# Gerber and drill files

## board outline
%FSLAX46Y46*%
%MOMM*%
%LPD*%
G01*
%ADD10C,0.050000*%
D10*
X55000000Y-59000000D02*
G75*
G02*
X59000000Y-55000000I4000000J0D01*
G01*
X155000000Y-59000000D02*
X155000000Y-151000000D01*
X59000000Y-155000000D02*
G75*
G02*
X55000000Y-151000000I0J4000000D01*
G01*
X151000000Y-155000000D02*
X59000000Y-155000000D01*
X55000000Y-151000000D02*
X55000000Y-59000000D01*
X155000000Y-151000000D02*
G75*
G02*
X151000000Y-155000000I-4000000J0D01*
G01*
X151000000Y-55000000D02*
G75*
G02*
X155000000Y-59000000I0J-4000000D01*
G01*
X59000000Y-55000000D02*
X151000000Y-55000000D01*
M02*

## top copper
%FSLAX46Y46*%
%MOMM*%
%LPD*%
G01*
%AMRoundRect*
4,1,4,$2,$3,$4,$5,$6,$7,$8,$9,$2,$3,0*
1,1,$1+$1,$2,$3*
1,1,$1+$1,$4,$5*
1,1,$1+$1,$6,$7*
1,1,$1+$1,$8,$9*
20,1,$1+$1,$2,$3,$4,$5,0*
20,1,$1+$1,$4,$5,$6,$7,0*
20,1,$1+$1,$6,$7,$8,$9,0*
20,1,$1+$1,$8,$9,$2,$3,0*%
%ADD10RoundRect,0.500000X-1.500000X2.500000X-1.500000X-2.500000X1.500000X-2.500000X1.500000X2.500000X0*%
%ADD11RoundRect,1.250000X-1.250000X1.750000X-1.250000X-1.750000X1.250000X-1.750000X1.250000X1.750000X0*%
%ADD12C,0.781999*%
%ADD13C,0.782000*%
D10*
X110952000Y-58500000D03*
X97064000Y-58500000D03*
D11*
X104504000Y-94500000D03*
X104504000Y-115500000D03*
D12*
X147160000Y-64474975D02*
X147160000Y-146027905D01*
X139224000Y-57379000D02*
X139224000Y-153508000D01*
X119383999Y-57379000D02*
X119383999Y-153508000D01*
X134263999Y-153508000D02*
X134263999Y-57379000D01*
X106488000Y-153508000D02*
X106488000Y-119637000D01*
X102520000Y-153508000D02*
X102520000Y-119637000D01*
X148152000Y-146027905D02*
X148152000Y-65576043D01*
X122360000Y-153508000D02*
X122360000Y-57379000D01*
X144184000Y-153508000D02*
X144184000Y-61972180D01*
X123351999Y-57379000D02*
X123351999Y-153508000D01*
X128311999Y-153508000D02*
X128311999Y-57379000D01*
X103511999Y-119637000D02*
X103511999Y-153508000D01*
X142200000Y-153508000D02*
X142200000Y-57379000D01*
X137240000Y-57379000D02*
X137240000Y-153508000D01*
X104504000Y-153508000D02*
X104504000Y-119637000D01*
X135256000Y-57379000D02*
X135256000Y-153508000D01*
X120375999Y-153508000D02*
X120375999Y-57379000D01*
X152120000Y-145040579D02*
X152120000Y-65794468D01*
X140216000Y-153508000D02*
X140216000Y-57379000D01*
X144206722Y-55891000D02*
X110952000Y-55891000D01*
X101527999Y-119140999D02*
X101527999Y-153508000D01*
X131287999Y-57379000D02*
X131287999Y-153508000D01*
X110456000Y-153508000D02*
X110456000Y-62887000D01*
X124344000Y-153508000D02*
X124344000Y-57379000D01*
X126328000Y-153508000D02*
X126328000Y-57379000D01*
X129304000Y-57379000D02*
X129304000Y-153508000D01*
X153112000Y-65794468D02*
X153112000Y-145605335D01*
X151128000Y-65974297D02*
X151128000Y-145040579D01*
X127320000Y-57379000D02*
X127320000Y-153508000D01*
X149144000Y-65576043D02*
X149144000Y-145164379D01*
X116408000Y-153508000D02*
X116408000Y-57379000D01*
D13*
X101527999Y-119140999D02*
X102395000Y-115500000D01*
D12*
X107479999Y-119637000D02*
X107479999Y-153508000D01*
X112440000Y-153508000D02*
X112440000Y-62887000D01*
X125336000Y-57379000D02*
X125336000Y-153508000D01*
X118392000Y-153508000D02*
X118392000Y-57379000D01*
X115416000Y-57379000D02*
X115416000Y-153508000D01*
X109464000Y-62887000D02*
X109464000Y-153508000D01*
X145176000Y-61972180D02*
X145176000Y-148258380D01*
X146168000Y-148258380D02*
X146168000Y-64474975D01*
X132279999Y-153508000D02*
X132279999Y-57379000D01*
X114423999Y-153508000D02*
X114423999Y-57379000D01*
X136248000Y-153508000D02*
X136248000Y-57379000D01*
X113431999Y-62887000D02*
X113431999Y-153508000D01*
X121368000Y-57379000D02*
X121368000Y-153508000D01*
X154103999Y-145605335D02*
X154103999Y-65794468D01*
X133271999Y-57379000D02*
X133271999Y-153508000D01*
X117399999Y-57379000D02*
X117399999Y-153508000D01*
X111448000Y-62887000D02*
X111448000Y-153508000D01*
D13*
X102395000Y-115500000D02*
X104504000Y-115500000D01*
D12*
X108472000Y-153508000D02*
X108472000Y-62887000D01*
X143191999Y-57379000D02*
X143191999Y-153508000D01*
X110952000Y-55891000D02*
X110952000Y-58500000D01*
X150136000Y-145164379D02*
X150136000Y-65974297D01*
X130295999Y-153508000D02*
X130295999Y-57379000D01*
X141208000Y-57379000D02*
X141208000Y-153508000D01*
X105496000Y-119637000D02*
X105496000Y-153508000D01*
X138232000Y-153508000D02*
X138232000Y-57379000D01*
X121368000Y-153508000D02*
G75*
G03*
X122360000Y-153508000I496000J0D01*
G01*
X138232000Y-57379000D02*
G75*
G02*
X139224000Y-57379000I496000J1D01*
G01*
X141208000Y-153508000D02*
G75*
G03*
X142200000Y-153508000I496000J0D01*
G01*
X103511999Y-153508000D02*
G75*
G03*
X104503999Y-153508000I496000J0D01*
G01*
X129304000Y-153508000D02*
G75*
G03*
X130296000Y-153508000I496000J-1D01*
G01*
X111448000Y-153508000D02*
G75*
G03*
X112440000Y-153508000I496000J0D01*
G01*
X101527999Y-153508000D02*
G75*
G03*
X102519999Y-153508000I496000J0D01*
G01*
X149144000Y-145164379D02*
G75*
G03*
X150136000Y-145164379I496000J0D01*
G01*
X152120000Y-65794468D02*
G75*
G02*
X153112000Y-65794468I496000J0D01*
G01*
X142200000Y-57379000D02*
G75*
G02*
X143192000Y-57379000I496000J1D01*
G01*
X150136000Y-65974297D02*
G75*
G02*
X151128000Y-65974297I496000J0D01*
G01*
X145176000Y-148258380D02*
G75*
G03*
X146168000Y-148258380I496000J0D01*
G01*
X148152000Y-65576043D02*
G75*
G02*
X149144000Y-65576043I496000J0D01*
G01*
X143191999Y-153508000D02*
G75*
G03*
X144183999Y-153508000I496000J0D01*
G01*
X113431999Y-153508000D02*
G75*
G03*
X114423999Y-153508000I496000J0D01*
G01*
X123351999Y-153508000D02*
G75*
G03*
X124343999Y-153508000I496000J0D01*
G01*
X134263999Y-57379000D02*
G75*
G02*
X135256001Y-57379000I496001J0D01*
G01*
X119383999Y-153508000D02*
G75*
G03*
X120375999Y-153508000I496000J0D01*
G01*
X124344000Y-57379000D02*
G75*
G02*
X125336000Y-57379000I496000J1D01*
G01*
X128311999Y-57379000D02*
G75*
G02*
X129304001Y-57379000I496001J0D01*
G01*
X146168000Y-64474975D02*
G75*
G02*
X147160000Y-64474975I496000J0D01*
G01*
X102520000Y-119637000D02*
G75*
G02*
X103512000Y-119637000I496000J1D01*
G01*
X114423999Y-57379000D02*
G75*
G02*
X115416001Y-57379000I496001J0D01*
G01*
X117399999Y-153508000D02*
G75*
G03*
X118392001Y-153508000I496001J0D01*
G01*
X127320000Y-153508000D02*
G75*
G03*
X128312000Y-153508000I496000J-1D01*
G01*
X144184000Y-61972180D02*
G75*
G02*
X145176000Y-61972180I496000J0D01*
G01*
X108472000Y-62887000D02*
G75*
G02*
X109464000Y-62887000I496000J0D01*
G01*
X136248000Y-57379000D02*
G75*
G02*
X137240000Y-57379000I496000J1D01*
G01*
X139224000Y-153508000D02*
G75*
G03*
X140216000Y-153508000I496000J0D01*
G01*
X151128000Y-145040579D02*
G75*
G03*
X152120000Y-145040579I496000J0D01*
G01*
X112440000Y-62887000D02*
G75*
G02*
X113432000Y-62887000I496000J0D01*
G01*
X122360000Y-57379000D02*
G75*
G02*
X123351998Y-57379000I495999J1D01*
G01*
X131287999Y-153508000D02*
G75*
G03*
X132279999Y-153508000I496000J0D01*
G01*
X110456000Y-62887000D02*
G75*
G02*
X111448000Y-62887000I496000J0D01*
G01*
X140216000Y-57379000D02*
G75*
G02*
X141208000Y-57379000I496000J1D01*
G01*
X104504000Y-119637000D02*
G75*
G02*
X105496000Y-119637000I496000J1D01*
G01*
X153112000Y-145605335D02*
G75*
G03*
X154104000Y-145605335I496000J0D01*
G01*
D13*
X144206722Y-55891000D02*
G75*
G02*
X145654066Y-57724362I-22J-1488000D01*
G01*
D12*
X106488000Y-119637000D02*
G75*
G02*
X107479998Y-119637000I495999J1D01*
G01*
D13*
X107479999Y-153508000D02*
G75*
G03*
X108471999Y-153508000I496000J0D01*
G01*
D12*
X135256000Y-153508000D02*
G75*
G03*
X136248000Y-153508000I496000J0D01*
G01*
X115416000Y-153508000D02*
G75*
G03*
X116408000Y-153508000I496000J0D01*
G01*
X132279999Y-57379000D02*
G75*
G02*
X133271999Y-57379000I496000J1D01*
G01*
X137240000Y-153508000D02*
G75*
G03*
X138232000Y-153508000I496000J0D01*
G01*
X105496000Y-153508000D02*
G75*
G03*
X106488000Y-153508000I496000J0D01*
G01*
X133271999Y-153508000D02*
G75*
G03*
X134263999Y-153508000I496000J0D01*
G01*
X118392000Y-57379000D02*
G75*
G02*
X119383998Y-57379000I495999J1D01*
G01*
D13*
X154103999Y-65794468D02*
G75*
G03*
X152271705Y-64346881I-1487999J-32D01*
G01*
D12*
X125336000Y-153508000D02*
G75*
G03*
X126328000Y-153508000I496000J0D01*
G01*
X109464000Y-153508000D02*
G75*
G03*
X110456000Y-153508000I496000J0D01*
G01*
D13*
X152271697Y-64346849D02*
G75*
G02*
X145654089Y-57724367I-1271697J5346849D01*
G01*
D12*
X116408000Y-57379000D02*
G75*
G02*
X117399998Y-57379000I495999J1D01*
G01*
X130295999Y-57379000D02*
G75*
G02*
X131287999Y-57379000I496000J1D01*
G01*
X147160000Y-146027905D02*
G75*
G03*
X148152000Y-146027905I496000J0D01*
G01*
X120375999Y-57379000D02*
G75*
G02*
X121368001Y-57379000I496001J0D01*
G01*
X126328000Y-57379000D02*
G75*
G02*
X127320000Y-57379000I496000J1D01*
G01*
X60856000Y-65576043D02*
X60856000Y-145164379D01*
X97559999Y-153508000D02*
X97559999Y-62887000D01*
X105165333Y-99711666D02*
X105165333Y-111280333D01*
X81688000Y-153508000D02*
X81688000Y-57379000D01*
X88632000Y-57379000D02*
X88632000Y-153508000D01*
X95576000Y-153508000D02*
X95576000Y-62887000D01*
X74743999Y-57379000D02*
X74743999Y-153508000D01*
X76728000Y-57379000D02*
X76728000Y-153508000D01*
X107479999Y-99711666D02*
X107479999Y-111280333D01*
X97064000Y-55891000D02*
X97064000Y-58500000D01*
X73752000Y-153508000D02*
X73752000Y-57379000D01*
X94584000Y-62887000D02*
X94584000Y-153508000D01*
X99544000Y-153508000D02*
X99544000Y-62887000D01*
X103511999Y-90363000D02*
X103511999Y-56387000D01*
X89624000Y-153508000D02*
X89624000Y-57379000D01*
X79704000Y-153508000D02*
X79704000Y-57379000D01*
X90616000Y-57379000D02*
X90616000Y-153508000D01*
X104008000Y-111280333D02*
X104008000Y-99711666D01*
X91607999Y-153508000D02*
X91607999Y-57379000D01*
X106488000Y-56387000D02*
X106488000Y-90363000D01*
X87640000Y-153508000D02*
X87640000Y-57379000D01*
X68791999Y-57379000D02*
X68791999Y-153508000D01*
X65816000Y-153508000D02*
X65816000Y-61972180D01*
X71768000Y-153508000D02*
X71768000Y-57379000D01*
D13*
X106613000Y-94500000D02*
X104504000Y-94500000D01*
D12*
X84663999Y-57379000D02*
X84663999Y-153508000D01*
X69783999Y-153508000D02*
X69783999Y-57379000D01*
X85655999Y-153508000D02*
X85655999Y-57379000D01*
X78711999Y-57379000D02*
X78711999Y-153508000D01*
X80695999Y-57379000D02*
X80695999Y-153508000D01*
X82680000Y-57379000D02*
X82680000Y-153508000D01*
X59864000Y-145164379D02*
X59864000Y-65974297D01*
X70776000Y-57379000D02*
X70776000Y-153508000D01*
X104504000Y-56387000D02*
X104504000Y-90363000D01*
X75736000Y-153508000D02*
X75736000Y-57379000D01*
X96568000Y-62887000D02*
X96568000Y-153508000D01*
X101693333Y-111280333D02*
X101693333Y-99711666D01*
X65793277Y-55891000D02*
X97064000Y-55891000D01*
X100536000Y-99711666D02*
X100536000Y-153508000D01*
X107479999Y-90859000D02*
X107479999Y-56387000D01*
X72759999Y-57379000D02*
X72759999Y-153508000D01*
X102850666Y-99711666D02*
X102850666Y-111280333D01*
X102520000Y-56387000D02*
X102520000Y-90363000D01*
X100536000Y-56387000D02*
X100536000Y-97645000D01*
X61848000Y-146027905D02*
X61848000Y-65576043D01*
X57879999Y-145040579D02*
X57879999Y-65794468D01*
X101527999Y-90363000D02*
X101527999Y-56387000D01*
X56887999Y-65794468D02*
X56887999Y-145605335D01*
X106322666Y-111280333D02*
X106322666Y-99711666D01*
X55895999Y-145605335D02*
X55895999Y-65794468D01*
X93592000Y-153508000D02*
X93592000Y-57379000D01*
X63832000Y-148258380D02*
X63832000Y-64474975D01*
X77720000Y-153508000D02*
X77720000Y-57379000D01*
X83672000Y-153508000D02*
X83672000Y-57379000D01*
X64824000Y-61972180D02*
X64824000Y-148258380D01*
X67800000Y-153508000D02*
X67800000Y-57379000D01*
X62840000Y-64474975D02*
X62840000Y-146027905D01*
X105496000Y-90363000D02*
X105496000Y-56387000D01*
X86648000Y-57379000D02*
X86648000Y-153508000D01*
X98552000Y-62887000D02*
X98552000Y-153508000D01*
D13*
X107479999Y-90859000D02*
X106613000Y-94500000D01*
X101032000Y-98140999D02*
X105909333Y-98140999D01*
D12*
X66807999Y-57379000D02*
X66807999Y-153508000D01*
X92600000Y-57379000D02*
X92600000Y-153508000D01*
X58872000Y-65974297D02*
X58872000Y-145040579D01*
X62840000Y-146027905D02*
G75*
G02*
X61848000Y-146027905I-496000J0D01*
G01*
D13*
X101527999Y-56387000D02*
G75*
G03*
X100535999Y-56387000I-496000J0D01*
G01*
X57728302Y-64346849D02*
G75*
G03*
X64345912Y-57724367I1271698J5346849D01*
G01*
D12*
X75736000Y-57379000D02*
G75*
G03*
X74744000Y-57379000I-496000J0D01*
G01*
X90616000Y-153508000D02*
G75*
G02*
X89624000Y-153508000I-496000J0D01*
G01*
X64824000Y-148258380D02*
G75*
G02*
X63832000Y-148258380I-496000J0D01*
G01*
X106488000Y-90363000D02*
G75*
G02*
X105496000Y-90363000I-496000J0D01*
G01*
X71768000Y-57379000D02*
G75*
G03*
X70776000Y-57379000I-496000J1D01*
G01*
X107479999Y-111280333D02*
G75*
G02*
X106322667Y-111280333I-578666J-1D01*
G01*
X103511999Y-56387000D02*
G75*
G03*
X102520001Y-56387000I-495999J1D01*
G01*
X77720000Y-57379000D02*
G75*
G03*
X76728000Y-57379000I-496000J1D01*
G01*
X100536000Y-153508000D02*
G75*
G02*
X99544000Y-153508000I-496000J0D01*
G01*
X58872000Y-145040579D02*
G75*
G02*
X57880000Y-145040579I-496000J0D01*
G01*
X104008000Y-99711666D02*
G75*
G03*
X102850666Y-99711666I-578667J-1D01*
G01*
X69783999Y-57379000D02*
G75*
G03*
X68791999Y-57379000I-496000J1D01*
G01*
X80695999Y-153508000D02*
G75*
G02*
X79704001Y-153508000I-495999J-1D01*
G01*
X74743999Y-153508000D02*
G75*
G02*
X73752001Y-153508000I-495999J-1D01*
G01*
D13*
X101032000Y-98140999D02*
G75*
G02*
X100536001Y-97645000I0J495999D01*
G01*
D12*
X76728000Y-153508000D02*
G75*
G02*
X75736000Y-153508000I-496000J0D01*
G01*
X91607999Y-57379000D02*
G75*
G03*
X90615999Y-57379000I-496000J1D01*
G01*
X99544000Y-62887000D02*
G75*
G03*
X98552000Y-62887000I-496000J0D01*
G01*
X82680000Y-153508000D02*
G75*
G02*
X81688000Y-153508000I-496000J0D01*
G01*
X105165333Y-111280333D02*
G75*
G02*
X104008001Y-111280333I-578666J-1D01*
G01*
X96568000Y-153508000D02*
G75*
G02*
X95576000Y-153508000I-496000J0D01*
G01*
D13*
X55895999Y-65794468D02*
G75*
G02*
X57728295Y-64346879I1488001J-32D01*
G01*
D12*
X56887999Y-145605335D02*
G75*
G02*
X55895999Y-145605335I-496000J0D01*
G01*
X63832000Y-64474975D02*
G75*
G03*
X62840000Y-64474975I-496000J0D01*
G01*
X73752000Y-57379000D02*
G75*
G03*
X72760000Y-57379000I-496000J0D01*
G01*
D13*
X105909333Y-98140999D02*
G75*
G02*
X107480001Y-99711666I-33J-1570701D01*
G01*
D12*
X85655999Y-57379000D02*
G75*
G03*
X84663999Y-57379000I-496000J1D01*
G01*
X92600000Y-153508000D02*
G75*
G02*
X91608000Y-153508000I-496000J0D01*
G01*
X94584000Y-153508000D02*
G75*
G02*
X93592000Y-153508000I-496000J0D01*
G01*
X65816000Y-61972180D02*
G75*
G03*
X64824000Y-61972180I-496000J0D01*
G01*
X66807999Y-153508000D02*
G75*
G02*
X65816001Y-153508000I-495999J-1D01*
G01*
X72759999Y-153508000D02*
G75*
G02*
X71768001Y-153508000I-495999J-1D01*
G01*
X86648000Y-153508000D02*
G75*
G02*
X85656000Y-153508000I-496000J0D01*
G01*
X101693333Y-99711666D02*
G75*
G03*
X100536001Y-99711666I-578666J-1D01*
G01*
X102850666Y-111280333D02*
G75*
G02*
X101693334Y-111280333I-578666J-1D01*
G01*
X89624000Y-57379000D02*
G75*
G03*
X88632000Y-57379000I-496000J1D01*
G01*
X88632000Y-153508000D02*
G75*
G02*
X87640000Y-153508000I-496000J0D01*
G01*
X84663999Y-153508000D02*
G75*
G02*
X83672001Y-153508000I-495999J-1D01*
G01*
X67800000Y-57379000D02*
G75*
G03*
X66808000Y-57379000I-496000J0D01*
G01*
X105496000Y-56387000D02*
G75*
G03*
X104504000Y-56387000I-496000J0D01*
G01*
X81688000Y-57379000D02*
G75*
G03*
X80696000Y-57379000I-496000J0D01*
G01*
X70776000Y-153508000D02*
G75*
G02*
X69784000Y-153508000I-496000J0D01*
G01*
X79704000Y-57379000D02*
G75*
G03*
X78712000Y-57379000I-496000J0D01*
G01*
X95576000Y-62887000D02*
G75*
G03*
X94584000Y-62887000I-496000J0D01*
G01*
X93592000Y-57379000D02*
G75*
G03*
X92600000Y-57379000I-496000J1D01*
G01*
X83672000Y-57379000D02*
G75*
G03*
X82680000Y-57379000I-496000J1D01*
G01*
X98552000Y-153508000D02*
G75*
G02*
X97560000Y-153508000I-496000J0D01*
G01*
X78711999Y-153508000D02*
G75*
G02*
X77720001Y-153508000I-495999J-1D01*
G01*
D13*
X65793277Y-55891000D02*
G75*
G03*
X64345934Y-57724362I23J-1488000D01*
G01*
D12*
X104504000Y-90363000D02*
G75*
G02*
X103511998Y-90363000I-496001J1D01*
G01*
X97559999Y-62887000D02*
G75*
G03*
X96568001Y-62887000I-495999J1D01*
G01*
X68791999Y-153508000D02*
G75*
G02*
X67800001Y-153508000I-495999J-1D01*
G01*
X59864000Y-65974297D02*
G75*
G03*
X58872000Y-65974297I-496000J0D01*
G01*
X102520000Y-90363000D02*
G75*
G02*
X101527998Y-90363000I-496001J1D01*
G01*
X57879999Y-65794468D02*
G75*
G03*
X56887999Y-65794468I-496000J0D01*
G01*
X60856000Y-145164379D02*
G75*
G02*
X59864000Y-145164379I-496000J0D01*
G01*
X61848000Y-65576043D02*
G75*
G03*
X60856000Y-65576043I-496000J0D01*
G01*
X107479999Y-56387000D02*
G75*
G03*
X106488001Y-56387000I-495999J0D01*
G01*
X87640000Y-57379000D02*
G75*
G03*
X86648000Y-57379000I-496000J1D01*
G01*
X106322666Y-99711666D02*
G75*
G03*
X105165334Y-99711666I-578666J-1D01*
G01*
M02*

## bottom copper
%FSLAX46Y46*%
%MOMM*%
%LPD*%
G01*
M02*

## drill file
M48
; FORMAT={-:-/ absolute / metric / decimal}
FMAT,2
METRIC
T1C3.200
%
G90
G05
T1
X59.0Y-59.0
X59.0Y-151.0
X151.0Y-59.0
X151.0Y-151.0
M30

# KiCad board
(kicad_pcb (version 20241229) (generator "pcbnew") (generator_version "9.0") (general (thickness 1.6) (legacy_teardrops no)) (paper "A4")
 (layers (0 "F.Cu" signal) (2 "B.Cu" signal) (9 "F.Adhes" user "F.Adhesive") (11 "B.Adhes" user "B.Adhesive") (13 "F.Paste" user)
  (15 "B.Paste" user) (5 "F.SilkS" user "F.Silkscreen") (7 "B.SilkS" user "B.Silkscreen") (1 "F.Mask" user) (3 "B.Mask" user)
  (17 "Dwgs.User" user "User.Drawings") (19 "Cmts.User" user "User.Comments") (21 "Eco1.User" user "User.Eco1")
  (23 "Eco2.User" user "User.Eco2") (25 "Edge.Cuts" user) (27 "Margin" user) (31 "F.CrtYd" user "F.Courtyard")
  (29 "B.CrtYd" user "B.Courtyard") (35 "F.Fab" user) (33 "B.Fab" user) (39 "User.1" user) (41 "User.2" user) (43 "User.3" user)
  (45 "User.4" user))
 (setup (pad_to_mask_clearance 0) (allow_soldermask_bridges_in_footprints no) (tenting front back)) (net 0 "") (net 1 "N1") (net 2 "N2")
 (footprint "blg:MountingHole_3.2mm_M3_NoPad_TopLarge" (layer "F.Cu") (at 151 59)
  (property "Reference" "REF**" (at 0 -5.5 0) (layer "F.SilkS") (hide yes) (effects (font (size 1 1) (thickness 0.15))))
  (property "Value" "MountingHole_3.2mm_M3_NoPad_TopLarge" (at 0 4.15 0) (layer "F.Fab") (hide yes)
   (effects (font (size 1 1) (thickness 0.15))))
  (pad "" np_thru_hole circle (at 0 0) (size 7.6 7.6) (drill 3.2) (layers) (zone_connect 2)))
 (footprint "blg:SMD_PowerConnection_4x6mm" (layer "F.Cu") (at 110.952 58.5 -90)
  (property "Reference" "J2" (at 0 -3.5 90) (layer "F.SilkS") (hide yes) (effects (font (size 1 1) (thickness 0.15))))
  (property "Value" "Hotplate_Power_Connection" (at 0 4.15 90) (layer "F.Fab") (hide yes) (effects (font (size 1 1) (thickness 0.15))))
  (pad "1" smd roundrect (at 0 0 270) (size 6 4) (layers "F.Cu" "F.Mask" "F.Paste") (roundrect_rratio 0.125) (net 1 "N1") (zone_connect 2)))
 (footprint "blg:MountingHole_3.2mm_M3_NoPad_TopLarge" (layer "F.Cu") (at 59 151)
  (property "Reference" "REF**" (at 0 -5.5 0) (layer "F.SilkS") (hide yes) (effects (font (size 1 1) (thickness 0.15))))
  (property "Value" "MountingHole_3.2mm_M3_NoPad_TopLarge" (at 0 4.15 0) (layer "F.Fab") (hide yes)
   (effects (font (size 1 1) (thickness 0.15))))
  (pad "" np_thru_hole circle (at 0 0) (size 7.6 7.6) (drill 3.2) (layers) (zone_connect 2)))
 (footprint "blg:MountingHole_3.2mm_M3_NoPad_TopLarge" (layer "F.Cu") (at 151 151)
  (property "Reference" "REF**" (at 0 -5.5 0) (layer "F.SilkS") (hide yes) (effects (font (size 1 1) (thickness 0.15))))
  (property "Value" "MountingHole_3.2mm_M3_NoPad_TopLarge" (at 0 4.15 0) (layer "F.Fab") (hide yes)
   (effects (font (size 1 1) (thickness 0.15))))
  (pad "" np_thru_hole circle (at 0 0) (size 7.6 7.6) (drill 3.2) (layers) (zone_connect 2)))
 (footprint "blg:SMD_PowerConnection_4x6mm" (layer "F.Cu") (at 97.064 58.5 -90)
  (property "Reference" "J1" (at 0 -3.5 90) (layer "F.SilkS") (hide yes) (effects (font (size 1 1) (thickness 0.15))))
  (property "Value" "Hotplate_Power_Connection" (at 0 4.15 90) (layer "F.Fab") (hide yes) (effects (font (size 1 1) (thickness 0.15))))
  (pad "1" smd roundrect (at 0 0 270) (size 6 4) (layers "F.Cu" "F.Mask" "F.Paste") (roundrect_rratio 0.125) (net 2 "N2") (zone_connect 2)))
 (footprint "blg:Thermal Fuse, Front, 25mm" (layer "F.Cu") (at 104.504 105 -90)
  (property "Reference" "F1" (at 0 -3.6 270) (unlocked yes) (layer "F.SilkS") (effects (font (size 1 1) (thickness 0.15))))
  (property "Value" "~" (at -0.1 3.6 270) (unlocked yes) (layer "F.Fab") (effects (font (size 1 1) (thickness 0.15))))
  (pad "1" smd roundrect (at -10.5 0 270) (size 6 5) (layers "F.Cu" "F.Mask") (roundrect_rratio 0.25) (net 2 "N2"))
  (pad "2" smd roundrect (at 10.5 0 270) (size 6 5) (layers "F.Cu" "F.Mask") (roundrect_rratio 0.25) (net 1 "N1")))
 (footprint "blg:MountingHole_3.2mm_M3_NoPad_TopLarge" (layer "F.Cu") (at 59 59)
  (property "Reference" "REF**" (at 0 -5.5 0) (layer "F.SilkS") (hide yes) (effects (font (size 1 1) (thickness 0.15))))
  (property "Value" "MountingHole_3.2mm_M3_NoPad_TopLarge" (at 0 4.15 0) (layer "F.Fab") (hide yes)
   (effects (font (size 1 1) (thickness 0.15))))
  (pad "" np_thru_hole circle (at 0 0) (size 7.6 7.6) (drill 3.2) (layers) (zone_connect 2)))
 (gr_arc (start 55 59) (mid 56.171573 56.171573) (end 59 55) (stroke (width 0.05) (type solid)) (layer "Edge.Cuts"))
 (gr_line (start 155 59) (end 155 151) (stroke (width 0.05) (type default)) (layer "Edge.Cuts"))
 (gr_arc (start 59 155) (mid 56.171573 153.828427) (end 55 151) (stroke (width 0.05) (type solid)) (layer "Edge.Cuts"))
 (gr_line (start 151 155) (end 59 155) (stroke (width 0.05) (type default)) (layer "Edge.Cuts"))
 (gr_line (start 55 151) (end 55 59) (stroke (width 0.05) (type default)) (layer "Edge.Cuts"))
 (gr_arc (start 155 151) (mid 153.828427 153.828427) (end 151 155) (stroke (width 0.05) (type solid)) (layer "Edge.Cuts"))
 (gr_arc (start 151 55) (mid 153.828427 56.171573) (end 155 59) (stroke (width 0.05) (type solid)) (layer "Edge.Cuts"))
 (gr_line (start 59 55) (end 151 55) (stroke (width 0.05) (type default)) (layer "Edge.Cuts"))
 (segment (start 147.16 64.474975) (end 147.16 146.027905) (width 0.781999) (layer "F.Cu") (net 1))
 (segment (start 139.224 57.379) (end 139.224 153.508) (width 0.781999) (layer "F.Cu") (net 1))
 (segment (start 119.383999 57.379) (end 119.383999 153.508) (width 0.781999) (layer "F.Cu") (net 1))
 (segment (start 134.263999 153.508) (end 134.263999 57.379) (width 0.781999) (layer "F.Cu") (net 1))
 (segment (start 106.488 153.508) (end 106.488 119.637) (width 0.781999) (layer "F.Cu") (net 1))
 (segment (start 102.52 153.508) (end 102.52 119.637) (width 0.781999) (layer "F.Cu") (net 1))
 (segment (start 148.152 146.027905) (end 148.152 65.576043) (width 0.781999) (layer "F.Cu") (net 1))
 (segment (start 122.36 153.508) (end 122.36 57.379) (width 0.781999) (layer "F.Cu") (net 1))
 (segment (start 144.184 153.508) (end 144.184 61.97218) (width 0.781999) (layer "F.Cu") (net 1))
 (segment (start 123.351999 57.379) (end 123.351999 153.508) (width 0.781999) (layer "F.Cu") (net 1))
 (segment (start 128.311999 153.508) (end 128.311999 57.379) (width 0.781999) (layer "F.Cu") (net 1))
 (segment (start 103.511999 119.637) (end 103.511999 153.508) (width 0.781999) (layer "F.Cu") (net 1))
 (segment (start 142.2 153.508) (end 142.2 57.379) (width 0.781999) (layer "F.Cu") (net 1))
 (segment (start 137.24 57.379) (end 137.24 153.508) (width 0.781999) (layer "F.Cu") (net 1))
 (segment (start 104.504 153.508) (end 104.504 119.637) (width 0.781999) (layer "F.Cu") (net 1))
 (segment (start 135.256 57.379) (end 135.256 153.508) (width 0.781999) (layer "F.Cu") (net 1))
 (segment (start 120.375999 153.508) (end 120.375999 57.379) (width 0.781999) (layer "F.Cu") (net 1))
 (segment (start 152.12 145.040579) (end 152.12 65.794468) (width 0.781999) (layer "F.Cu") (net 1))
 (segment (start 140.216 153.508) (end 140.216 57.379) (width 0.781999) (layer "F.Cu") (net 1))
 (segment (start 144.206722 55.891) (end 110.952 55.891) (width 0.781999) (layer "F.Cu") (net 1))
 (segment (start 101.527999 119.140999) (end 101.527999 153.508) (width 0.781999) (layer "F.Cu") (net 1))
 (segment (start 131.287999 57.379) (end 131.287999 153.508) (width 0.781999) (layer "F.Cu") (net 1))
 (segment (start 110.456 153.508) (end 110.456 62.887) (width 0.781999) (layer "F.Cu") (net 1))
 (segment (start 124.344 153.508) (end 124.344 57.379) (width 0.781999) (layer "F.Cu") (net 1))
 (segment (start 126.328 153.508) (end 126.328 57.379) (width 0.781999) (layer "F.Cu") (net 1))
 (segment (start 129.304 57.379) (end 129.304 153.508) (width 0.781999) (layer "F.Cu") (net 1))
 (segment (start 153.112 65.794468) (end 153.112 145.605335) (width 0.781999) (layer "F.Cu") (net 1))
 (segment (start 151.128 65.974297) (end 151.128 145.040579) (width 0.781999) (layer "F.Cu") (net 1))
 (segment (start 127.32 57.379) (end 127.32 153.508) (width 0.781999) (layer "F.Cu") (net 1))
 (segment (start 149.144 65.576043) (end 149.144 145.164379) (width 0.781999) (layer "F.Cu") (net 1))
 (segment (start 116.408 153.508) (end 116.408 57.379) (width 0.781999) (layer "F.Cu") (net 1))
 (segment (start 101.527999 119.140999) (end 102.395 115.5) (width 0.782) (layer "F.Cu") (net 1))
 (segment (start 107.479999 119.637) (end 107.479999 153.508) (width 0.781999) (layer "F.Cu") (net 1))
 (segment (start 112.44 153.508) (end 112.44 62.887) (width 0.781999) (layer "F.Cu") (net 1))
 (segment (start 125.336 57.379) (end 125.336 153.508) (width 0.781999) (layer "F.Cu") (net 1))
 (segment (start 118.392 153.508) (end 118.392 57.379) (width 0.781999) (layer "F.Cu") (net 1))
 (segment (start 115.416 57.379) (end 115.416 153.508) (width 0.781999) (layer "F.Cu") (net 1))
 (segment (start 109.464 62.887) (end 109.464 153.508) (width 0.781999) (layer "F.Cu") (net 1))
 (segment (start 145.176 61.97218) (end 145.176 148.25838) (width 0.781999) (layer "F.Cu") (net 1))
 (segment (start 146.168 148.25838) (end 146.168 64.474975) (width 0.781999) (layer "F.Cu") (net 1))
 (segment (start 132.279999 153.508) (end 132.279999 57.379) (width 0.781999) (layer "F.Cu") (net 1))
 (segment (start 114.423999 153.508) (end 114.423999 57.379) (width 0.781999) (layer "F.Cu") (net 1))
 (segment (start 136.248 153.508) (end 136.248 57.379) (width 0.781999) (layer "F.Cu") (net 1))
 (segment (start 113.431999 62.887) (end 113.431999 153.508) (width 0.781999) (layer "F.Cu") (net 1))
 (segment (start 121.368 57.379) (end 121.368 153.508) (width 0.781999) (layer "F.Cu") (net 1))
 (segment (start 154.103999 145.605335) (end 154.103999 65.794468) (width 0.781999) (layer "F.Cu") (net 1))
 (segment (start 133.271999 57.379) (end 133.271999 153.508) (width 0.781999) (layer "F.Cu") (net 1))
 (segment (start 117.399999 57.379) (end 117.399999 153.508) (width 0.781999) (layer "F.Cu") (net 1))
 (segment (start 111.448 62.887) (end 111.448 153.508) (width 0.781999) (layer "F.Cu") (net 1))
 (segment (start 102.395 115.5) (end 104.504 115.5) (width 0.782) (layer "F.Cu") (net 1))
 (segment (start 108.472 153.508) (end 108.472 62.887) (width 0.781999) (layer "F.Cu") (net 1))
 (segment (start 143.191999 57.379) (end 143.191999 153.508) (width 0.781999) (layer "F.Cu") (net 1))
 (segment (start 110.952 55.891) (end 110.952 58.5) (width 0.781999) (layer "F.Cu") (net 1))
 (segment (start 150.136 145.164379) (end 150.136 65.974297) (width 0.781999) (layer "F.Cu") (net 1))
 (segment (start 130.295999 153.508) (end 130.295999 57.379) (width 0.781999) (layer "F.Cu") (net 1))
 (segment (start 141.208 57.379) (end 141.208 153.508) (width 0.781999) (layer "F.Cu") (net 1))
 (segment (start 105.496 119.637) (end 105.496 153.508) (width 0.781999) (layer "F.Cu") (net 1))
 (segment (start 138.232 153.508) (end 138.232 57.379) (width 0.781999) (layer "F.Cu") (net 1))
 (arc (start 121.368 153.508) (mid 121.864 154.004) (end 122.36 153.508) (width 0.781999) (layer "F.Cu") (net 1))
 (arc (start 138.232 57.379) (mid 138.727999 56.882999) (end 139.224 57.379) (width 0.781999) (layer "F.Cu") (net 1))
 (arc (start 141.208 153.508) (mid 141.704 154.004) (end 142.2 153.508) (width 0.781999) (layer "F.Cu") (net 1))
 (arc (start 103.511999 153.508) (mid 104.008 154.004) (end 104.504 153.508) (width 0.781999) (layer "F.Cu") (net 1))
 (arc (start 129.304 153.508) (mid 129.8 154.004) (end 130.295999 153.508) (width 0.781999) (layer "F.Cu") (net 1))
 (arc (start 111.448 153.508) (mid 111.944 154.004) (end 112.44 153.508) (width 0.781999) (layer "F.Cu") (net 1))
 (arc (start 101.527999 153.508) (mid 102.023999 154.004) (end 102.52 153.508) (width 0.781999) (layer "F.Cu") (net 1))
 (arc (start 149.144 145.164379) (mid 149.64 145.660379) (end 150.136 145.164379) (width 0.781999) (layer "F.Cu") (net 1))
 (arc (start 152.12 65.794468) (mid 152.616 65.298468) (end 153.112 65.794468) (width 0.781999) (layer "F.Cu") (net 1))
 (arc (start 142.2 57.379) (mid 142.696 56.882999) (end 143.191999 57.379) (width 0.781999) (layer "F.Cu") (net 1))
 (arc (start 150.136 65.974297) (mid 150.631999 65.478297) (end 151.128 65.974297) (width 0.781999) (layer "F.Cu") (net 1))
 (arc (start 145.176 148.25838) (mid 145.672 148.75438) (end 146.168 148.25838) (width 0.781999) (layer "F.Cu") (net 1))
 (arc (start 148.152 65.576043) (mid 148.648 65.080043) (end 149.144 65.576043) (width 0.781999) (layer "F.Cu") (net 1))
 (arc (start 143.191999 153.508) (mid 143.688 154.004) (end 144.184 153.508) (width 0.781999) (layer "F.Cu") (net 1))
 (arc (start 113.431999 153.508) (mid 113.928 154.004) (end 114.423999 153.508) (width 0.781999) (layer "F.Cu") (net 1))
 (arc (start 123.351999 153.508) (mid 123.848 154.004) (end 124.344 153.508) (width 0.781999) (layer "F.Cu") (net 1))
 (arc (start 134.263999 57.379) (mid 134.76 56.882999) (end 135.256 57.379) (width 0.781999) (layer "F.Cu") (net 1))
 (arc (start 119.383999 153.508) (mid 119.88 154.004) (end 120.375999 153.508) (width 0.781999) (layer "F.Cu") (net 1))
 (arc (start 124.344 57.379) (mid 124.839999 56.882999) (end 125.336 57.379) (width 0.781999) (layer "F.Cu") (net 1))
 (arc (start 128.311999 57.379) (mid 128.808 56.882999) (end 129.304 57.379) (width 0.781999) (layer "F.Cu") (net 1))
 (arc (start 146.168 64.474975) (mid 146.664 63.978975) (end 147.16 64.474975) (width 0.781999) (layer "F.Cu") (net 1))
 (arc (start 102.52 119.637) (mid 103.015999 119.140999) (end 103.511999 119.637) (width 0.781999) (layer "F.Cu") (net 1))
 (arc (start 114.423999 57.379) (mid 114.919999 56.882999) (end 115.416 57.379) (width 0.781999) (layer "F.Cu") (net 1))
 (arc (start 117.399999 153.508) (mid 117.896 154.004) (end 118.392 153.508) (width 0.781999) (layer "F.Cu") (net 1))
 (arc (start 127.32 153.508) (mid 127.815999 154.004) (end 128.311999 153.508) (width 0.781999) (layer "F.Cu") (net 1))
 (arc (start 144.184 61.97218) (mid 144.68 61.47618) (end 145.176 61.97218) (width 0.781999) (layer "F.Cu") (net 1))
 (arc (start 108.472 62.887) (mid 108.967999 62.391) (end 109.464 62.887) (width 0.781999) (layer "F.Cu") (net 1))
 (arc (start 136.248 57.379) (mid 136.744 56.882999) (end 137.24 57.379) (width 0.781999) (layer "F.Cu") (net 1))
 (arc (start 139.224 153.508) (mid 139.719999 154.004) (end 140.216 153.508) (width 0.781999) (layer "F.Cu") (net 1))
 (arc (start 151.128 145.040579) (mid 151.623999 145.536579) (end 152.12 145.040579) (width 0.781999) (layer "F.Cu") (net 1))
 (arc (start 112.44 62.887) (mid 112.936 62.391) (end 113.431999 62.887) (width 0.781999) (layer "F.Cu") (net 1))
 (arc (start 122.36 57.379) (mid 122.856 56.882999) (end 123.351999 57.379) (width 0.781999) (layer "F.Cu") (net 1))
 (arc (start 131.287999 153.508) (mid 131.783999 154.004) (end 132.279999 153.508) (width 0.781999) (layer "F.Cu") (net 1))
 (arc (start 110.456 62.887) (mid 110.952 62.391) (end 111.448 62.887) (width 0.781999) (layer "F.Cu") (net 1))
 (arc (start 140.216 57.379) (mid 140.712 56.882999) (end 141.208 57.379) (width 0.781999) (layer "F.Cu") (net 1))
 (arc (start 104.504 119.637) (mid 105 119.140999) (end 105.496 119.637) (width 0.781999) (layer "F.Cu") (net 1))
 (arc (start 153.112 145.605335) (mid 153.608 146.101335) (end 154.103999 145.605335) (width 0.781999) (layer "F.Cu") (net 1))
 (arc (start 144.206722 55.891) (mid 145.374637 56.456981) (end 145.654087 57.724367) (width 0.782) (layer "F.Cu") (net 1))
 (arc (start 106.488 119.637) (mid 106.984 119.140999) (end 107.479999 119.637) (width 0.781999) (layer "F.Cu") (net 1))
 (arc (start 107.479999 153.508) (mid 107.975999 154.004) (end 108.472 153.508) (width 0.782) (layer "F.Cu") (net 1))
 (arc (start 135.256 153.508) (mid 135.751999 154.004) (end 136.248 153.508) (width 0.781999) (layer "F.Cu") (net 1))
 (arc (start 115.416 153.508) (mid 115.912 154.004) (end 116.408 153.508) (width 0.781999) (layer "F.Cu") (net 1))
 (arc (start 132.279999 57.379) (mid 132.776 56.882999) (end 133.271999 57.379) (width 0.781999) (layer "F.Cu") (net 1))
 (arc (start 137.24 153.508) (mid 137.736 154.004) (end 138.232 153.508) (width 0.781999) (layer "F.Cu") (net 1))
 (arc (start 105.496 153.508) (mid 105.991999 154.004) (end 106.488 153.508) (width 0.781999) (layer "F.Cu") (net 1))
 (arc (start 133.271999 153.508) (mid 133.768 154.004) (end 134.263999 153.508) (width 0.781999) (layer "F.Cu") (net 1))
 (arc (start 118.392 57.379) (mid 118.887999 56.882999) (end 119.383999 57.379) (width 0.781999) (layer "F.Cu") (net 1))
 (arc (start 154.103999 65.794468) (mid 153.692767 64.767474) (end 152.271697 64.346849) (width 0.782) (layer "F.Cu") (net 1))
 (arc (start 125.336 153.508) (mid 125.832 154.004) (end 126.328 153.508) (width 0.781999) (layer "F.Cu") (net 1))
 (arc (start 109.464 153.508) (mid 109.96 154.004) (end 110.456 153.508) (width 0.781999) (layer "F.Cu") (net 1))
 (arc (start 152.271697 64.346849) (mid 147.112311 62.884828) (end 145.654087 57.724367) (width 0.782) (layer "F.Cu") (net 1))
 (arc (start 116.408 57.379) (mid 116.904 56.882999) (end 117.399999 57.379) (width 0.781999) (layer "F.Cu") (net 1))
 (arc (start 130.295999 57.379) (mid 130.792 56.882999) (end 131.287999 57.379) (width 0.781999) (layer "F.Cu") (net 1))
 (arc (start 147.16 146.027905) (mid 147.655999 146.523905) (end 148.152 146.027905) (width 0.781999) (layer "F.Cu") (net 1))
 (arc (start 120.375999 57.379) (mid 120.872 56.882999) (end 121.368 57.379) (width 0.781999) (layer "F.Cu") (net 1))
 (arc (start 126.328 57.379) (mid 126.824 56.882999) (end 127.32 57.379) (width 0.781999) (layer "F.Cu") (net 1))
 (segment (start 60.856 65.576043) (end 60.856 145.164379) (width 0.781999) (layer "F.Cu") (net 2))
 (segment (start 97.559999 153.508) (end 97.559999 62.887) (width 0.781999) (layer "F.Cu") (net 2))
 (segment (start 105.165333 99.711666) (end 105.165333 111.280333) (width 0.781999) (layer "F.Cu") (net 2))
 (segment (start 81.688 153.508) (end 81.688 57.379) (width 0.781999) (layer "F.Cu") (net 2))
 (segment (start 88.632 57.379) (end 88.632 153.508) (width 0.781999) (layer "F.Cu") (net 2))
 (segment (start 95.576 153.508) (end 95.576 62.887) (width 0.781999) (layer "F.Cu") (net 2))
 (segment (start 74.743999 57.379) (end 74.743999 153.508) (width 0.781999) (layer "F.Cu") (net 2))
 (segment (start 76.728 57.379) (end 76.728 153.508) (width 0.781999) (layer "F.Cu") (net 2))
 (segment (start 107.479999 99.711666) (end 107.479999 111.280333) (width 0.781999) (layer "F.Cu") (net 2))
 (segment (start 97.064 55.891) (end 97.064 58.5) (width 0.781999) (layer "F.Cu") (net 2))
 (segment (start 73.752 153.508) (end 73.752 57.379) (width 0.781999) (layer "F.Cu") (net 2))
 (segment (start 94.584 62.887) (end 94.584 153.508) (width 0.781999) (layer "F.Cu") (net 2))
 (segment (start 99.544 153.508) (end 99.544 62.887) (width 0.781999) (layer "F.Cu") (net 2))
 (segment (start 103.511999 90.363) (end 103.511999 56.387) (width 0.781999) (layer "F.Cu") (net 2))
 (segment (start 89.624 153.508) (end 89.624 57.379) (width 0.781999) (layer "F.Cu") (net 2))
 (segment (start 79.704 153.508) (end 79.704 57.379) (width 0.781999) (layer "F.Cu") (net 2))
 (segment (start 90.616 57.379) (end 90.616 153.508) (width 0.781999) (layer "F.Cu") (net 2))
 (segment (start 104.008 111.280333) (end 104.008 99.711666) (width 0.781999) (layer "F.Cu") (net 2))
 (segment (start 91.607999 153.508) (end 91.607999 57.379) (width 0.781999) (layer "F.Cu") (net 2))
 (segment (start 106.488 56.387) (end 106.488 90.363) (width 0.781999) (layer "F.Cu") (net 2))
 (segment (start 87.64 153.508) (end 87.64 57.379) (width 0.781999) (layer "F.Cu") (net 2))
 (segment (start 68.791999 57.379) (end 68.791999 153.508) (width 0.781999) (layer "F.Cu") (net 2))
 (segment (start 65.816 153.508) (end 65.816 61.97218) (width 0.781999) (layer "F.Cu") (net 2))
 (segment (start 71.768 153.508) (end 71.768 57.379) (width 0.781999) (layer "F.Cu") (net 2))
 (segment (start 106.613 94.5) (end 104.504 94.5) (width 0.782) (layer "F.Cu") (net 2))
 (segment (start 84.663999 57.379) (end 84.663999 153.508) (width 0.781999) (layer "F.Cu") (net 2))
 (segment (start 69.783999 153.508) (end 69.783999 57.379) (width 0.781999) (layer "F.Cu") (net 2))
 (segment (start 85.655999 153.508) (end 85.655999 57.379) (width 0.781999) (layer "F.Cu") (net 2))
 (segment (start 78.711999 57.379) (end 78.711999 153.508) (width 0.781999) (layer "F.Cu") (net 2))
 (segment (start 80.695999 57.379) (end 80.695999 153.508) (width 0.781999) (layer "F.Cu") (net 2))
 (segment (start 82.68 57.379) (end 82.68 153.508) (width 0.781999) (layer "F.Cu") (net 2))
 (segment (start 59.864 145.164379) (end 59.864 65.974297) (width 0.781999) (layer "F.Cu") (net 2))
 (segment (start 70.776 57.379) (end 70.776 153.508) (width 0.781999) (layer "F.Cu") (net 2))
 (segment (start 104.504 56.387) (end 104.504 90.363) (width 0.781999) (layer "F.Cu") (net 2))
 (segment (start 75.736 153.508) (end 75.736 57.379) (width 0.781999) (layer "F.Cu") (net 2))
 (segment (start 96.568 62.887) (end 96.568 153.508) (width 0.781999) (layer "F.Cu") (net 2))
 (segment (start 101.693333 111.280333) (end 101.693333 99.711666) (width 0.781999) (layer "F.Cu") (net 2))
 (segment (start 65.793277 55.891) (end 97.064 55.891) (width 0.781999) (layer "F.Cu") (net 2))
 (segment (start 100.536 99.711666) (end 100.536 153.508) (width 0.781999) (layer "F.Cu") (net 2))
 (segment (start 107.479999 90.859) (end 107.479999 56.387) (width 0.781999) (layer "F.Cu") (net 2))
 (segment (start 72.759999 57.379) (end 72.759999 153.508) (width 0.781999) (layer "F.Cu") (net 2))
 (segment (start 102.850666 99.711666) (end 102.850666 111.280333) (width 0.781999) (layer "F.Cu") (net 2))
 (segment (start 102.52 56.387) (end 102.52 90.363) (width 0.781999) (layer "F.Cu") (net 2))
 (segment (start 100.536 56.387) (end 100.536 97.645) (width 0.781999) (layer "F.Cu") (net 2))
 (segment (start 61.848 146.027905) (end 61.848 65.576043) (width 0.781999) (layer "F.Cu") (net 2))
 (segment (start 57.879999 145.040579) (end 57.879999 65.794468) (width 0.781999) (layer "F.Cu") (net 2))
 (segment (start 101.527999 90.363) (end 101.527999 56.387) (width 0.781999) (layer "F.Cu") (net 2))
 (segment (start 56.887999 65.794468) (end 56.887999 145.605335) (width 0.781999) (layer "F.Cu") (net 2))
 (segment (start 106.322666 111.280333) (end 106.322666 99.711666) (width 0.781999) (layer "F.Cu") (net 2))
 (segment (start 55.895999 145.605335) (end 55.895999 65.794468) (width 0.781999) (layer "F.Cu") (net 2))
 (segment (start 93.592 153.508) (end 93.592 57.379) (width 0.781999) (layer "F.Cu") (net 2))
 (segment (start 63.832 148.25838) (end 63.832 64.474975) (width 0.781999) (layer "F.Cu") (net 2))
 (segment (start 77.72 153.508) (end 77.72 57.379) (width 0.781999) (layer "F.Cu") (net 2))
 (segment (start 83.672 153.508) (end 83.672 57.379) (width 0.781999) (layer "F.Cu") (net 2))
 (segment (start 64.824 61.97218) (end 64.824 148.25838) (width 0.781999) (layer "F.Cu") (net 2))
 (segment (start 67.8 153.508) (end 67.8 57.379) (width 0.781999) (layer "F.Cu") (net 2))
 (segment (start 62.84 64.474975) (end 62.84 146.027905) (width 0.781999) (layer "F.Cu") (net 2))
 (segment (start 105.496 90.363) (end 105.496 56.387) (width 0.781999) (layer "F.Cu") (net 2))
 (segment (start 86.648 57.379) (end 86.648 153.508) (width 0.781999) (layer "F.Cu") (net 2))
 (segment (start 98.552 62.887) (end 98.552 153.508) (width 0.781999) (layer "F.Cu") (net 2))
 (segment (start 107.479999 90.859) (end 106.613 94.5) (width 0.782) (layer "F.Cu") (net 2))
 (segment (start 101.032 98.140999) (end 105.909333 98.140999) (width 0.782) (layer "F.Cu") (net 2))
 (segment (start 66.807999 57.379) (end 66.807999 153.508) (width 0.781999) (layer "F.Cu") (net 2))
 (segment (start 92.6 57.379) (end 92.6 153.508) (width 0.781999) (layer "F.Cu") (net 2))
 (segment (start 58.872 65.974297) (end 58.872 145.040579) (width 0.781999) (layer "F.Cu") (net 2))
 (arc (start 62.84 146.027905) (mid 62.343999 146.523905) (end 61.848 146.027905) (width 0.781999) (layer "F.Cu") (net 2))
 (arc (start 101.527999 56.387) (mid 101.032 55.891) (end 100.535999 56.387) (width 0.782) (layer "F.Cu") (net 2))
 (arc (start 57.728302 64.346849) (mid 62.887688 62.884828) (end 64.345912 57.724367) (width 0.782) (layer "F.Cu") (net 2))
 (arc (start 75.736 57.379) (mid 75.24 56.882999) (end 74.743999 57.379) (width 0.781999) (layer "F.Cu") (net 2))
 (arc (start 90.616 153.508) (mid 90.119999 154.004) (end 89.624 153.508) (width 0.781999) (layer "F.Cu") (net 2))
 (arc (start 64.824 148.25838) (mid 64.328 148.75438) (end 63.832 148.25838) (width 0.781999) (layer "F.Cu") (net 2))
 (arc (start 106.488 90.363) (mid 105.991999 90.859) (end 105.496 90.363) (width 0.781999) (layer "F.Cu") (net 2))
 (arc (start 71.768 57.379) (mid 71.272 56.882999) (end 70.776 57.379) (width 0.781999) (layer "F.Cu") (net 2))
 (arc (start 107.479999 111.280333) (mid 106.901333 111.859) (end 106.322666 111.280333) (width 0.781999) (layer "F.Cu") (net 2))
 (arc (start 103.511999 56.387) (mid 103.015999 55.891) (end 102.52 56.387) (width 0.781999) (layer "F.Cu") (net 2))
 (arc (start 77.72 57.379) (mid 77.224 56.882999) (end 76.728 57.379) (width 0.781999) (layer "F.Cu") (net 2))
 (arc (start 100.536 153.508) (mid 100.039999 154.004) (end 99.544 153.508) (width 0.781999) (layer "F.Cu") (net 2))
 (arc (start 58.872 145.040579) (mid 58.376 145.536579) (end 57.879999 145.040579) (width 0.781999) (layer "F.Cu") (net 2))
 (arc (start 104.008 99.711666) (mid 103.429333 99.133) (end 102.850666 99.711666) (width 0.781999) (layer "F.Cu") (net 2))
 (arc (start 69.783999 57.379) (mid 69.288 56.882999) (end 68.791999 57.379) (width 0.781999) (layer "F.Cu") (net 2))
 (arc (start 80.695999 153.508) (mid 80.199999 154.004) (end 79.704 153.508) (width 0.781999) (layer "F.Cu") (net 2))
 (arc (start 74.743999 153.508) (mid 74.247999 154.004) (end 73.752 153.508) (width 0.781999) (layer "F.Cu") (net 2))
 (arc (start 101.032 98.140999) (mid 100.681275 97.995724) (end 100.536 97.645) (width 0.782) (layer "F.Cu") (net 2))
 (arc (start 76.728 153.508) (mid 76.232 154.004) (end 75.736 153.508) (width 0.781999) (layer "F.Cu") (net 2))
 (arc (start 91.607999 57.379) (mid 91.112 56.882999) (end 90.616 57.379) (width 0.781999) (layer "F.Cu") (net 2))
 (arc (start 99.544 62.887) (mid 99.048 62.391) (end 98.552 62.887) (width 0.781999) (layer "F.Cu") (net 2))
 (arc (start 82.68 153.508) (mid 82.184 154.004) (end 81.688 153.508) (width 0.781999) (layer "F.Cu") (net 2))
 (arc (start 105.165333 111.280333) (mid 104.586666 111.859) (end 104.008 111.280333) (width 0.781999) (layer "F.Cu") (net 2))
 (arc (start 96.568 153.508) (mid 96.071999 154.004) (end 95.576 153.508) (width 0.781999) (layer "F.Cu") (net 2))
 (arc (start 55.895999 65.794468) (mid 56.307232 64.767474) (end 57.728302 64.346849) (width 0.782) (layer "F.Cu") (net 2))
 (arc (start 56.887999 145.605335) (mid 56.391999 146.101335) (end 55.895999 145.605335) (width 0.781999) (layer "F.Cu") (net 2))
 (arc (start 63.832 64.474975) (mid 63.336 63.978975) (end 62.84 64.474975) (width 0.781999) (layer "F.Cu") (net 2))
 (arc (start 73.752 57.379) (mid 73.256 56.882999) (end 72.759999 57.379) (width 0.781999) (layer "F.Cu") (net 2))
 (arc (start 105.909333 98.140999) (mid 107.019962 98.601037) (end 107.479999 99.711666) (width 0.782) (layer "F.Cu") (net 2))
 (arc (start 85.655999 57.379) (mid 85.16 56.882999) (end 84.663999 57.379) (width 0.781999) (layer "F.Cu") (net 2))
 (arc (start 92.6 153.508) (mid 92.103999 154.004) (end 91.607999 153.508) (width 0.781999) (layer "F.Cu") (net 2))
 (arc (start 94.584 153.508) (mid 94.088 154.004) (end 93.592 153.508) (width 0.781999) (layer "F.Cu") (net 2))
 (arc (start 65.816 61.97218) (mid 65.32 61.47618) (end 64.824 61.97218) (width 0.781999) (layer "F.Cu") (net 2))
 (arc (start 66.807999 153.508) (mid 66.312 154.004) (end 65.816 153.508) (width 0.781999) (layer "F.Cu") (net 2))
 (arc (start 72.759999 153.508) (mid 72.264 154.004) (end 71.768 153.508) (width 0.781999) (layer "F.Cu") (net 2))
 (arc (start 86.648 153.508) (mid 86.151999 154.004) (end 85.655999 153.508) (width 0.781999) (layer "F.Cu") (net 2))
 (arc (start 101.693333 99.711666) (mid 101.114666 99.133) (end 100.536 99.711666) (width 0.781999) (layer "F.Cu") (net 2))
 (arc (start 102.850666 111.280333) (mid 102.272 111.859) (end 101.693333 111.280333) (width 0.781999) (layer "F.Cu") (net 2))
 (arc (start 89.624 57.379) (mid 89.128 56.882999) (end 88.632 57.379) (width 0.781999) (layer "F.Cu") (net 2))
 (arc (start 88.632 153.508) (mid 88.136 154.004) (end 87.64 153.508) (width 0.781999) (layer "F.Cu") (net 2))
 (arc (start 84.663999 153.508) (mid 84.167999 154.004) (end 83.672 153.508) (width 0.781999) (layer "F.Cu") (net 2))
 (arc (start 67.8 57.379) (mid 67.304 56.882999) (end 66.807999 57.379) (width 0.781999) (layer "F.Cu") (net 2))
 (arc (start 105.496 56.387) (mid 105 55.891) (end 104.504 56.387) (width 0.781999) (layer "F.Cu") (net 2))
 (arc (start 81.688 57.379) (mid 81.192 56.882999) (end 80.695999 57.379) (width 0.781999) (layer "F.Cu") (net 2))
 (arc (start 70.776 153.508) (mid 70.28 154.004) (end 69.783999 153.508) (width 0.781999) (layer "F.Cu") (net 2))
 (arc (start 79.704 57.379) (mid 79.208 56.882999) (end 78.711999 57.379) (width 0.781999) (layer "F.Cu") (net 2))
 (arc (start 95.576 62.887) (mid 95.08 62.391) (end 94.584 62.887) (width 0.781999) (layer "F.Cu") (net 2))
 (arc (start 93.592 57.379) (mid 93.096 56.882999) (end 92.6 57.379) (width 0.781999) (layer "F.Cu") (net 2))
 (arc (start 83.672 57.379) (mid 83.176 56.882999) (end 82.68 57.379) (width 0.781999) (layer "F.Cu") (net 2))
 (arc (start 98.552 153.508) (mid 98.056 154.004) (end 97.559999 153.508) (width 0.781999) (layer "F.Cu") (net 2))
 (arc (start 78.711999 153.508) (mid 78.216 154.004) (end 77.72 153.508) (width 0.781999) (layer "F.Cu") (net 2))
 (arc (start 65.793277 55.891) (mid 64.625362 56.456981) (end 64.345912 57.724367) (width 0.782) (layer "F.Cu") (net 2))
 (arc (start 104.504 90.363) (mid 104.008 90.859) (end 103.511999 90.363) (width 0.781999) (layer "F.Cu") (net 2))
 (arc (start 97.559999 62.887) (mid 97.064 62.391) (end 96.568 62.887) (width 0.781999) (layer "F.Cu") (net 2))
 (arc (start 68.791999 153.508) (mid 68.295999 154.004) (end 67.8 153.508) (width 0.781999) (layer "F.Cu") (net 2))
 (arc (start 59.864 65.974297) (mid 59.367999 65.478297) (end 58.872 65.974297) (width 0.781999) (layer "F.Cu") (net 2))
 (arc (start 102.52 90.363) (mid 102.023999 90.859) (end 101.527999 90.363) (width 0.781999) (layer "F.Cu") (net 2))
 (arc (start 57.879999 65.794468) (mid 57.384 65.298468) (end 56.887999 65.794468) (width 0.781999) (layer "F.Cu") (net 2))
 (arc (start 60.856 145.164379) (mid 60.36 145.660379) (end 59.864 145.164379) (width 0.781999) (layer "F.Cu") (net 2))
 (arc (start 61.848 65.576043) (mid 61.352 65.080043) (end 60.856 65.576043) (width 0.781999) (layer "F.Cu") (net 2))
 (arc (start 107.479999 56.387) (mid 106.984 55.891) (end 106.488 56.387) (width 0.781999) (layer "F.Cu") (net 2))
 (arc (start 87.64 57.379) (mid 87.144 56.882999) (end 86.648 57.379) (width 0.781999) (layer "F.Cu") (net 2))
 (arc (start 106.322666 99.711666) (mid 105.743999 99.133) (end 105.165333 99.711666) (width 0.781999) (layer "F.Cu") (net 2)))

